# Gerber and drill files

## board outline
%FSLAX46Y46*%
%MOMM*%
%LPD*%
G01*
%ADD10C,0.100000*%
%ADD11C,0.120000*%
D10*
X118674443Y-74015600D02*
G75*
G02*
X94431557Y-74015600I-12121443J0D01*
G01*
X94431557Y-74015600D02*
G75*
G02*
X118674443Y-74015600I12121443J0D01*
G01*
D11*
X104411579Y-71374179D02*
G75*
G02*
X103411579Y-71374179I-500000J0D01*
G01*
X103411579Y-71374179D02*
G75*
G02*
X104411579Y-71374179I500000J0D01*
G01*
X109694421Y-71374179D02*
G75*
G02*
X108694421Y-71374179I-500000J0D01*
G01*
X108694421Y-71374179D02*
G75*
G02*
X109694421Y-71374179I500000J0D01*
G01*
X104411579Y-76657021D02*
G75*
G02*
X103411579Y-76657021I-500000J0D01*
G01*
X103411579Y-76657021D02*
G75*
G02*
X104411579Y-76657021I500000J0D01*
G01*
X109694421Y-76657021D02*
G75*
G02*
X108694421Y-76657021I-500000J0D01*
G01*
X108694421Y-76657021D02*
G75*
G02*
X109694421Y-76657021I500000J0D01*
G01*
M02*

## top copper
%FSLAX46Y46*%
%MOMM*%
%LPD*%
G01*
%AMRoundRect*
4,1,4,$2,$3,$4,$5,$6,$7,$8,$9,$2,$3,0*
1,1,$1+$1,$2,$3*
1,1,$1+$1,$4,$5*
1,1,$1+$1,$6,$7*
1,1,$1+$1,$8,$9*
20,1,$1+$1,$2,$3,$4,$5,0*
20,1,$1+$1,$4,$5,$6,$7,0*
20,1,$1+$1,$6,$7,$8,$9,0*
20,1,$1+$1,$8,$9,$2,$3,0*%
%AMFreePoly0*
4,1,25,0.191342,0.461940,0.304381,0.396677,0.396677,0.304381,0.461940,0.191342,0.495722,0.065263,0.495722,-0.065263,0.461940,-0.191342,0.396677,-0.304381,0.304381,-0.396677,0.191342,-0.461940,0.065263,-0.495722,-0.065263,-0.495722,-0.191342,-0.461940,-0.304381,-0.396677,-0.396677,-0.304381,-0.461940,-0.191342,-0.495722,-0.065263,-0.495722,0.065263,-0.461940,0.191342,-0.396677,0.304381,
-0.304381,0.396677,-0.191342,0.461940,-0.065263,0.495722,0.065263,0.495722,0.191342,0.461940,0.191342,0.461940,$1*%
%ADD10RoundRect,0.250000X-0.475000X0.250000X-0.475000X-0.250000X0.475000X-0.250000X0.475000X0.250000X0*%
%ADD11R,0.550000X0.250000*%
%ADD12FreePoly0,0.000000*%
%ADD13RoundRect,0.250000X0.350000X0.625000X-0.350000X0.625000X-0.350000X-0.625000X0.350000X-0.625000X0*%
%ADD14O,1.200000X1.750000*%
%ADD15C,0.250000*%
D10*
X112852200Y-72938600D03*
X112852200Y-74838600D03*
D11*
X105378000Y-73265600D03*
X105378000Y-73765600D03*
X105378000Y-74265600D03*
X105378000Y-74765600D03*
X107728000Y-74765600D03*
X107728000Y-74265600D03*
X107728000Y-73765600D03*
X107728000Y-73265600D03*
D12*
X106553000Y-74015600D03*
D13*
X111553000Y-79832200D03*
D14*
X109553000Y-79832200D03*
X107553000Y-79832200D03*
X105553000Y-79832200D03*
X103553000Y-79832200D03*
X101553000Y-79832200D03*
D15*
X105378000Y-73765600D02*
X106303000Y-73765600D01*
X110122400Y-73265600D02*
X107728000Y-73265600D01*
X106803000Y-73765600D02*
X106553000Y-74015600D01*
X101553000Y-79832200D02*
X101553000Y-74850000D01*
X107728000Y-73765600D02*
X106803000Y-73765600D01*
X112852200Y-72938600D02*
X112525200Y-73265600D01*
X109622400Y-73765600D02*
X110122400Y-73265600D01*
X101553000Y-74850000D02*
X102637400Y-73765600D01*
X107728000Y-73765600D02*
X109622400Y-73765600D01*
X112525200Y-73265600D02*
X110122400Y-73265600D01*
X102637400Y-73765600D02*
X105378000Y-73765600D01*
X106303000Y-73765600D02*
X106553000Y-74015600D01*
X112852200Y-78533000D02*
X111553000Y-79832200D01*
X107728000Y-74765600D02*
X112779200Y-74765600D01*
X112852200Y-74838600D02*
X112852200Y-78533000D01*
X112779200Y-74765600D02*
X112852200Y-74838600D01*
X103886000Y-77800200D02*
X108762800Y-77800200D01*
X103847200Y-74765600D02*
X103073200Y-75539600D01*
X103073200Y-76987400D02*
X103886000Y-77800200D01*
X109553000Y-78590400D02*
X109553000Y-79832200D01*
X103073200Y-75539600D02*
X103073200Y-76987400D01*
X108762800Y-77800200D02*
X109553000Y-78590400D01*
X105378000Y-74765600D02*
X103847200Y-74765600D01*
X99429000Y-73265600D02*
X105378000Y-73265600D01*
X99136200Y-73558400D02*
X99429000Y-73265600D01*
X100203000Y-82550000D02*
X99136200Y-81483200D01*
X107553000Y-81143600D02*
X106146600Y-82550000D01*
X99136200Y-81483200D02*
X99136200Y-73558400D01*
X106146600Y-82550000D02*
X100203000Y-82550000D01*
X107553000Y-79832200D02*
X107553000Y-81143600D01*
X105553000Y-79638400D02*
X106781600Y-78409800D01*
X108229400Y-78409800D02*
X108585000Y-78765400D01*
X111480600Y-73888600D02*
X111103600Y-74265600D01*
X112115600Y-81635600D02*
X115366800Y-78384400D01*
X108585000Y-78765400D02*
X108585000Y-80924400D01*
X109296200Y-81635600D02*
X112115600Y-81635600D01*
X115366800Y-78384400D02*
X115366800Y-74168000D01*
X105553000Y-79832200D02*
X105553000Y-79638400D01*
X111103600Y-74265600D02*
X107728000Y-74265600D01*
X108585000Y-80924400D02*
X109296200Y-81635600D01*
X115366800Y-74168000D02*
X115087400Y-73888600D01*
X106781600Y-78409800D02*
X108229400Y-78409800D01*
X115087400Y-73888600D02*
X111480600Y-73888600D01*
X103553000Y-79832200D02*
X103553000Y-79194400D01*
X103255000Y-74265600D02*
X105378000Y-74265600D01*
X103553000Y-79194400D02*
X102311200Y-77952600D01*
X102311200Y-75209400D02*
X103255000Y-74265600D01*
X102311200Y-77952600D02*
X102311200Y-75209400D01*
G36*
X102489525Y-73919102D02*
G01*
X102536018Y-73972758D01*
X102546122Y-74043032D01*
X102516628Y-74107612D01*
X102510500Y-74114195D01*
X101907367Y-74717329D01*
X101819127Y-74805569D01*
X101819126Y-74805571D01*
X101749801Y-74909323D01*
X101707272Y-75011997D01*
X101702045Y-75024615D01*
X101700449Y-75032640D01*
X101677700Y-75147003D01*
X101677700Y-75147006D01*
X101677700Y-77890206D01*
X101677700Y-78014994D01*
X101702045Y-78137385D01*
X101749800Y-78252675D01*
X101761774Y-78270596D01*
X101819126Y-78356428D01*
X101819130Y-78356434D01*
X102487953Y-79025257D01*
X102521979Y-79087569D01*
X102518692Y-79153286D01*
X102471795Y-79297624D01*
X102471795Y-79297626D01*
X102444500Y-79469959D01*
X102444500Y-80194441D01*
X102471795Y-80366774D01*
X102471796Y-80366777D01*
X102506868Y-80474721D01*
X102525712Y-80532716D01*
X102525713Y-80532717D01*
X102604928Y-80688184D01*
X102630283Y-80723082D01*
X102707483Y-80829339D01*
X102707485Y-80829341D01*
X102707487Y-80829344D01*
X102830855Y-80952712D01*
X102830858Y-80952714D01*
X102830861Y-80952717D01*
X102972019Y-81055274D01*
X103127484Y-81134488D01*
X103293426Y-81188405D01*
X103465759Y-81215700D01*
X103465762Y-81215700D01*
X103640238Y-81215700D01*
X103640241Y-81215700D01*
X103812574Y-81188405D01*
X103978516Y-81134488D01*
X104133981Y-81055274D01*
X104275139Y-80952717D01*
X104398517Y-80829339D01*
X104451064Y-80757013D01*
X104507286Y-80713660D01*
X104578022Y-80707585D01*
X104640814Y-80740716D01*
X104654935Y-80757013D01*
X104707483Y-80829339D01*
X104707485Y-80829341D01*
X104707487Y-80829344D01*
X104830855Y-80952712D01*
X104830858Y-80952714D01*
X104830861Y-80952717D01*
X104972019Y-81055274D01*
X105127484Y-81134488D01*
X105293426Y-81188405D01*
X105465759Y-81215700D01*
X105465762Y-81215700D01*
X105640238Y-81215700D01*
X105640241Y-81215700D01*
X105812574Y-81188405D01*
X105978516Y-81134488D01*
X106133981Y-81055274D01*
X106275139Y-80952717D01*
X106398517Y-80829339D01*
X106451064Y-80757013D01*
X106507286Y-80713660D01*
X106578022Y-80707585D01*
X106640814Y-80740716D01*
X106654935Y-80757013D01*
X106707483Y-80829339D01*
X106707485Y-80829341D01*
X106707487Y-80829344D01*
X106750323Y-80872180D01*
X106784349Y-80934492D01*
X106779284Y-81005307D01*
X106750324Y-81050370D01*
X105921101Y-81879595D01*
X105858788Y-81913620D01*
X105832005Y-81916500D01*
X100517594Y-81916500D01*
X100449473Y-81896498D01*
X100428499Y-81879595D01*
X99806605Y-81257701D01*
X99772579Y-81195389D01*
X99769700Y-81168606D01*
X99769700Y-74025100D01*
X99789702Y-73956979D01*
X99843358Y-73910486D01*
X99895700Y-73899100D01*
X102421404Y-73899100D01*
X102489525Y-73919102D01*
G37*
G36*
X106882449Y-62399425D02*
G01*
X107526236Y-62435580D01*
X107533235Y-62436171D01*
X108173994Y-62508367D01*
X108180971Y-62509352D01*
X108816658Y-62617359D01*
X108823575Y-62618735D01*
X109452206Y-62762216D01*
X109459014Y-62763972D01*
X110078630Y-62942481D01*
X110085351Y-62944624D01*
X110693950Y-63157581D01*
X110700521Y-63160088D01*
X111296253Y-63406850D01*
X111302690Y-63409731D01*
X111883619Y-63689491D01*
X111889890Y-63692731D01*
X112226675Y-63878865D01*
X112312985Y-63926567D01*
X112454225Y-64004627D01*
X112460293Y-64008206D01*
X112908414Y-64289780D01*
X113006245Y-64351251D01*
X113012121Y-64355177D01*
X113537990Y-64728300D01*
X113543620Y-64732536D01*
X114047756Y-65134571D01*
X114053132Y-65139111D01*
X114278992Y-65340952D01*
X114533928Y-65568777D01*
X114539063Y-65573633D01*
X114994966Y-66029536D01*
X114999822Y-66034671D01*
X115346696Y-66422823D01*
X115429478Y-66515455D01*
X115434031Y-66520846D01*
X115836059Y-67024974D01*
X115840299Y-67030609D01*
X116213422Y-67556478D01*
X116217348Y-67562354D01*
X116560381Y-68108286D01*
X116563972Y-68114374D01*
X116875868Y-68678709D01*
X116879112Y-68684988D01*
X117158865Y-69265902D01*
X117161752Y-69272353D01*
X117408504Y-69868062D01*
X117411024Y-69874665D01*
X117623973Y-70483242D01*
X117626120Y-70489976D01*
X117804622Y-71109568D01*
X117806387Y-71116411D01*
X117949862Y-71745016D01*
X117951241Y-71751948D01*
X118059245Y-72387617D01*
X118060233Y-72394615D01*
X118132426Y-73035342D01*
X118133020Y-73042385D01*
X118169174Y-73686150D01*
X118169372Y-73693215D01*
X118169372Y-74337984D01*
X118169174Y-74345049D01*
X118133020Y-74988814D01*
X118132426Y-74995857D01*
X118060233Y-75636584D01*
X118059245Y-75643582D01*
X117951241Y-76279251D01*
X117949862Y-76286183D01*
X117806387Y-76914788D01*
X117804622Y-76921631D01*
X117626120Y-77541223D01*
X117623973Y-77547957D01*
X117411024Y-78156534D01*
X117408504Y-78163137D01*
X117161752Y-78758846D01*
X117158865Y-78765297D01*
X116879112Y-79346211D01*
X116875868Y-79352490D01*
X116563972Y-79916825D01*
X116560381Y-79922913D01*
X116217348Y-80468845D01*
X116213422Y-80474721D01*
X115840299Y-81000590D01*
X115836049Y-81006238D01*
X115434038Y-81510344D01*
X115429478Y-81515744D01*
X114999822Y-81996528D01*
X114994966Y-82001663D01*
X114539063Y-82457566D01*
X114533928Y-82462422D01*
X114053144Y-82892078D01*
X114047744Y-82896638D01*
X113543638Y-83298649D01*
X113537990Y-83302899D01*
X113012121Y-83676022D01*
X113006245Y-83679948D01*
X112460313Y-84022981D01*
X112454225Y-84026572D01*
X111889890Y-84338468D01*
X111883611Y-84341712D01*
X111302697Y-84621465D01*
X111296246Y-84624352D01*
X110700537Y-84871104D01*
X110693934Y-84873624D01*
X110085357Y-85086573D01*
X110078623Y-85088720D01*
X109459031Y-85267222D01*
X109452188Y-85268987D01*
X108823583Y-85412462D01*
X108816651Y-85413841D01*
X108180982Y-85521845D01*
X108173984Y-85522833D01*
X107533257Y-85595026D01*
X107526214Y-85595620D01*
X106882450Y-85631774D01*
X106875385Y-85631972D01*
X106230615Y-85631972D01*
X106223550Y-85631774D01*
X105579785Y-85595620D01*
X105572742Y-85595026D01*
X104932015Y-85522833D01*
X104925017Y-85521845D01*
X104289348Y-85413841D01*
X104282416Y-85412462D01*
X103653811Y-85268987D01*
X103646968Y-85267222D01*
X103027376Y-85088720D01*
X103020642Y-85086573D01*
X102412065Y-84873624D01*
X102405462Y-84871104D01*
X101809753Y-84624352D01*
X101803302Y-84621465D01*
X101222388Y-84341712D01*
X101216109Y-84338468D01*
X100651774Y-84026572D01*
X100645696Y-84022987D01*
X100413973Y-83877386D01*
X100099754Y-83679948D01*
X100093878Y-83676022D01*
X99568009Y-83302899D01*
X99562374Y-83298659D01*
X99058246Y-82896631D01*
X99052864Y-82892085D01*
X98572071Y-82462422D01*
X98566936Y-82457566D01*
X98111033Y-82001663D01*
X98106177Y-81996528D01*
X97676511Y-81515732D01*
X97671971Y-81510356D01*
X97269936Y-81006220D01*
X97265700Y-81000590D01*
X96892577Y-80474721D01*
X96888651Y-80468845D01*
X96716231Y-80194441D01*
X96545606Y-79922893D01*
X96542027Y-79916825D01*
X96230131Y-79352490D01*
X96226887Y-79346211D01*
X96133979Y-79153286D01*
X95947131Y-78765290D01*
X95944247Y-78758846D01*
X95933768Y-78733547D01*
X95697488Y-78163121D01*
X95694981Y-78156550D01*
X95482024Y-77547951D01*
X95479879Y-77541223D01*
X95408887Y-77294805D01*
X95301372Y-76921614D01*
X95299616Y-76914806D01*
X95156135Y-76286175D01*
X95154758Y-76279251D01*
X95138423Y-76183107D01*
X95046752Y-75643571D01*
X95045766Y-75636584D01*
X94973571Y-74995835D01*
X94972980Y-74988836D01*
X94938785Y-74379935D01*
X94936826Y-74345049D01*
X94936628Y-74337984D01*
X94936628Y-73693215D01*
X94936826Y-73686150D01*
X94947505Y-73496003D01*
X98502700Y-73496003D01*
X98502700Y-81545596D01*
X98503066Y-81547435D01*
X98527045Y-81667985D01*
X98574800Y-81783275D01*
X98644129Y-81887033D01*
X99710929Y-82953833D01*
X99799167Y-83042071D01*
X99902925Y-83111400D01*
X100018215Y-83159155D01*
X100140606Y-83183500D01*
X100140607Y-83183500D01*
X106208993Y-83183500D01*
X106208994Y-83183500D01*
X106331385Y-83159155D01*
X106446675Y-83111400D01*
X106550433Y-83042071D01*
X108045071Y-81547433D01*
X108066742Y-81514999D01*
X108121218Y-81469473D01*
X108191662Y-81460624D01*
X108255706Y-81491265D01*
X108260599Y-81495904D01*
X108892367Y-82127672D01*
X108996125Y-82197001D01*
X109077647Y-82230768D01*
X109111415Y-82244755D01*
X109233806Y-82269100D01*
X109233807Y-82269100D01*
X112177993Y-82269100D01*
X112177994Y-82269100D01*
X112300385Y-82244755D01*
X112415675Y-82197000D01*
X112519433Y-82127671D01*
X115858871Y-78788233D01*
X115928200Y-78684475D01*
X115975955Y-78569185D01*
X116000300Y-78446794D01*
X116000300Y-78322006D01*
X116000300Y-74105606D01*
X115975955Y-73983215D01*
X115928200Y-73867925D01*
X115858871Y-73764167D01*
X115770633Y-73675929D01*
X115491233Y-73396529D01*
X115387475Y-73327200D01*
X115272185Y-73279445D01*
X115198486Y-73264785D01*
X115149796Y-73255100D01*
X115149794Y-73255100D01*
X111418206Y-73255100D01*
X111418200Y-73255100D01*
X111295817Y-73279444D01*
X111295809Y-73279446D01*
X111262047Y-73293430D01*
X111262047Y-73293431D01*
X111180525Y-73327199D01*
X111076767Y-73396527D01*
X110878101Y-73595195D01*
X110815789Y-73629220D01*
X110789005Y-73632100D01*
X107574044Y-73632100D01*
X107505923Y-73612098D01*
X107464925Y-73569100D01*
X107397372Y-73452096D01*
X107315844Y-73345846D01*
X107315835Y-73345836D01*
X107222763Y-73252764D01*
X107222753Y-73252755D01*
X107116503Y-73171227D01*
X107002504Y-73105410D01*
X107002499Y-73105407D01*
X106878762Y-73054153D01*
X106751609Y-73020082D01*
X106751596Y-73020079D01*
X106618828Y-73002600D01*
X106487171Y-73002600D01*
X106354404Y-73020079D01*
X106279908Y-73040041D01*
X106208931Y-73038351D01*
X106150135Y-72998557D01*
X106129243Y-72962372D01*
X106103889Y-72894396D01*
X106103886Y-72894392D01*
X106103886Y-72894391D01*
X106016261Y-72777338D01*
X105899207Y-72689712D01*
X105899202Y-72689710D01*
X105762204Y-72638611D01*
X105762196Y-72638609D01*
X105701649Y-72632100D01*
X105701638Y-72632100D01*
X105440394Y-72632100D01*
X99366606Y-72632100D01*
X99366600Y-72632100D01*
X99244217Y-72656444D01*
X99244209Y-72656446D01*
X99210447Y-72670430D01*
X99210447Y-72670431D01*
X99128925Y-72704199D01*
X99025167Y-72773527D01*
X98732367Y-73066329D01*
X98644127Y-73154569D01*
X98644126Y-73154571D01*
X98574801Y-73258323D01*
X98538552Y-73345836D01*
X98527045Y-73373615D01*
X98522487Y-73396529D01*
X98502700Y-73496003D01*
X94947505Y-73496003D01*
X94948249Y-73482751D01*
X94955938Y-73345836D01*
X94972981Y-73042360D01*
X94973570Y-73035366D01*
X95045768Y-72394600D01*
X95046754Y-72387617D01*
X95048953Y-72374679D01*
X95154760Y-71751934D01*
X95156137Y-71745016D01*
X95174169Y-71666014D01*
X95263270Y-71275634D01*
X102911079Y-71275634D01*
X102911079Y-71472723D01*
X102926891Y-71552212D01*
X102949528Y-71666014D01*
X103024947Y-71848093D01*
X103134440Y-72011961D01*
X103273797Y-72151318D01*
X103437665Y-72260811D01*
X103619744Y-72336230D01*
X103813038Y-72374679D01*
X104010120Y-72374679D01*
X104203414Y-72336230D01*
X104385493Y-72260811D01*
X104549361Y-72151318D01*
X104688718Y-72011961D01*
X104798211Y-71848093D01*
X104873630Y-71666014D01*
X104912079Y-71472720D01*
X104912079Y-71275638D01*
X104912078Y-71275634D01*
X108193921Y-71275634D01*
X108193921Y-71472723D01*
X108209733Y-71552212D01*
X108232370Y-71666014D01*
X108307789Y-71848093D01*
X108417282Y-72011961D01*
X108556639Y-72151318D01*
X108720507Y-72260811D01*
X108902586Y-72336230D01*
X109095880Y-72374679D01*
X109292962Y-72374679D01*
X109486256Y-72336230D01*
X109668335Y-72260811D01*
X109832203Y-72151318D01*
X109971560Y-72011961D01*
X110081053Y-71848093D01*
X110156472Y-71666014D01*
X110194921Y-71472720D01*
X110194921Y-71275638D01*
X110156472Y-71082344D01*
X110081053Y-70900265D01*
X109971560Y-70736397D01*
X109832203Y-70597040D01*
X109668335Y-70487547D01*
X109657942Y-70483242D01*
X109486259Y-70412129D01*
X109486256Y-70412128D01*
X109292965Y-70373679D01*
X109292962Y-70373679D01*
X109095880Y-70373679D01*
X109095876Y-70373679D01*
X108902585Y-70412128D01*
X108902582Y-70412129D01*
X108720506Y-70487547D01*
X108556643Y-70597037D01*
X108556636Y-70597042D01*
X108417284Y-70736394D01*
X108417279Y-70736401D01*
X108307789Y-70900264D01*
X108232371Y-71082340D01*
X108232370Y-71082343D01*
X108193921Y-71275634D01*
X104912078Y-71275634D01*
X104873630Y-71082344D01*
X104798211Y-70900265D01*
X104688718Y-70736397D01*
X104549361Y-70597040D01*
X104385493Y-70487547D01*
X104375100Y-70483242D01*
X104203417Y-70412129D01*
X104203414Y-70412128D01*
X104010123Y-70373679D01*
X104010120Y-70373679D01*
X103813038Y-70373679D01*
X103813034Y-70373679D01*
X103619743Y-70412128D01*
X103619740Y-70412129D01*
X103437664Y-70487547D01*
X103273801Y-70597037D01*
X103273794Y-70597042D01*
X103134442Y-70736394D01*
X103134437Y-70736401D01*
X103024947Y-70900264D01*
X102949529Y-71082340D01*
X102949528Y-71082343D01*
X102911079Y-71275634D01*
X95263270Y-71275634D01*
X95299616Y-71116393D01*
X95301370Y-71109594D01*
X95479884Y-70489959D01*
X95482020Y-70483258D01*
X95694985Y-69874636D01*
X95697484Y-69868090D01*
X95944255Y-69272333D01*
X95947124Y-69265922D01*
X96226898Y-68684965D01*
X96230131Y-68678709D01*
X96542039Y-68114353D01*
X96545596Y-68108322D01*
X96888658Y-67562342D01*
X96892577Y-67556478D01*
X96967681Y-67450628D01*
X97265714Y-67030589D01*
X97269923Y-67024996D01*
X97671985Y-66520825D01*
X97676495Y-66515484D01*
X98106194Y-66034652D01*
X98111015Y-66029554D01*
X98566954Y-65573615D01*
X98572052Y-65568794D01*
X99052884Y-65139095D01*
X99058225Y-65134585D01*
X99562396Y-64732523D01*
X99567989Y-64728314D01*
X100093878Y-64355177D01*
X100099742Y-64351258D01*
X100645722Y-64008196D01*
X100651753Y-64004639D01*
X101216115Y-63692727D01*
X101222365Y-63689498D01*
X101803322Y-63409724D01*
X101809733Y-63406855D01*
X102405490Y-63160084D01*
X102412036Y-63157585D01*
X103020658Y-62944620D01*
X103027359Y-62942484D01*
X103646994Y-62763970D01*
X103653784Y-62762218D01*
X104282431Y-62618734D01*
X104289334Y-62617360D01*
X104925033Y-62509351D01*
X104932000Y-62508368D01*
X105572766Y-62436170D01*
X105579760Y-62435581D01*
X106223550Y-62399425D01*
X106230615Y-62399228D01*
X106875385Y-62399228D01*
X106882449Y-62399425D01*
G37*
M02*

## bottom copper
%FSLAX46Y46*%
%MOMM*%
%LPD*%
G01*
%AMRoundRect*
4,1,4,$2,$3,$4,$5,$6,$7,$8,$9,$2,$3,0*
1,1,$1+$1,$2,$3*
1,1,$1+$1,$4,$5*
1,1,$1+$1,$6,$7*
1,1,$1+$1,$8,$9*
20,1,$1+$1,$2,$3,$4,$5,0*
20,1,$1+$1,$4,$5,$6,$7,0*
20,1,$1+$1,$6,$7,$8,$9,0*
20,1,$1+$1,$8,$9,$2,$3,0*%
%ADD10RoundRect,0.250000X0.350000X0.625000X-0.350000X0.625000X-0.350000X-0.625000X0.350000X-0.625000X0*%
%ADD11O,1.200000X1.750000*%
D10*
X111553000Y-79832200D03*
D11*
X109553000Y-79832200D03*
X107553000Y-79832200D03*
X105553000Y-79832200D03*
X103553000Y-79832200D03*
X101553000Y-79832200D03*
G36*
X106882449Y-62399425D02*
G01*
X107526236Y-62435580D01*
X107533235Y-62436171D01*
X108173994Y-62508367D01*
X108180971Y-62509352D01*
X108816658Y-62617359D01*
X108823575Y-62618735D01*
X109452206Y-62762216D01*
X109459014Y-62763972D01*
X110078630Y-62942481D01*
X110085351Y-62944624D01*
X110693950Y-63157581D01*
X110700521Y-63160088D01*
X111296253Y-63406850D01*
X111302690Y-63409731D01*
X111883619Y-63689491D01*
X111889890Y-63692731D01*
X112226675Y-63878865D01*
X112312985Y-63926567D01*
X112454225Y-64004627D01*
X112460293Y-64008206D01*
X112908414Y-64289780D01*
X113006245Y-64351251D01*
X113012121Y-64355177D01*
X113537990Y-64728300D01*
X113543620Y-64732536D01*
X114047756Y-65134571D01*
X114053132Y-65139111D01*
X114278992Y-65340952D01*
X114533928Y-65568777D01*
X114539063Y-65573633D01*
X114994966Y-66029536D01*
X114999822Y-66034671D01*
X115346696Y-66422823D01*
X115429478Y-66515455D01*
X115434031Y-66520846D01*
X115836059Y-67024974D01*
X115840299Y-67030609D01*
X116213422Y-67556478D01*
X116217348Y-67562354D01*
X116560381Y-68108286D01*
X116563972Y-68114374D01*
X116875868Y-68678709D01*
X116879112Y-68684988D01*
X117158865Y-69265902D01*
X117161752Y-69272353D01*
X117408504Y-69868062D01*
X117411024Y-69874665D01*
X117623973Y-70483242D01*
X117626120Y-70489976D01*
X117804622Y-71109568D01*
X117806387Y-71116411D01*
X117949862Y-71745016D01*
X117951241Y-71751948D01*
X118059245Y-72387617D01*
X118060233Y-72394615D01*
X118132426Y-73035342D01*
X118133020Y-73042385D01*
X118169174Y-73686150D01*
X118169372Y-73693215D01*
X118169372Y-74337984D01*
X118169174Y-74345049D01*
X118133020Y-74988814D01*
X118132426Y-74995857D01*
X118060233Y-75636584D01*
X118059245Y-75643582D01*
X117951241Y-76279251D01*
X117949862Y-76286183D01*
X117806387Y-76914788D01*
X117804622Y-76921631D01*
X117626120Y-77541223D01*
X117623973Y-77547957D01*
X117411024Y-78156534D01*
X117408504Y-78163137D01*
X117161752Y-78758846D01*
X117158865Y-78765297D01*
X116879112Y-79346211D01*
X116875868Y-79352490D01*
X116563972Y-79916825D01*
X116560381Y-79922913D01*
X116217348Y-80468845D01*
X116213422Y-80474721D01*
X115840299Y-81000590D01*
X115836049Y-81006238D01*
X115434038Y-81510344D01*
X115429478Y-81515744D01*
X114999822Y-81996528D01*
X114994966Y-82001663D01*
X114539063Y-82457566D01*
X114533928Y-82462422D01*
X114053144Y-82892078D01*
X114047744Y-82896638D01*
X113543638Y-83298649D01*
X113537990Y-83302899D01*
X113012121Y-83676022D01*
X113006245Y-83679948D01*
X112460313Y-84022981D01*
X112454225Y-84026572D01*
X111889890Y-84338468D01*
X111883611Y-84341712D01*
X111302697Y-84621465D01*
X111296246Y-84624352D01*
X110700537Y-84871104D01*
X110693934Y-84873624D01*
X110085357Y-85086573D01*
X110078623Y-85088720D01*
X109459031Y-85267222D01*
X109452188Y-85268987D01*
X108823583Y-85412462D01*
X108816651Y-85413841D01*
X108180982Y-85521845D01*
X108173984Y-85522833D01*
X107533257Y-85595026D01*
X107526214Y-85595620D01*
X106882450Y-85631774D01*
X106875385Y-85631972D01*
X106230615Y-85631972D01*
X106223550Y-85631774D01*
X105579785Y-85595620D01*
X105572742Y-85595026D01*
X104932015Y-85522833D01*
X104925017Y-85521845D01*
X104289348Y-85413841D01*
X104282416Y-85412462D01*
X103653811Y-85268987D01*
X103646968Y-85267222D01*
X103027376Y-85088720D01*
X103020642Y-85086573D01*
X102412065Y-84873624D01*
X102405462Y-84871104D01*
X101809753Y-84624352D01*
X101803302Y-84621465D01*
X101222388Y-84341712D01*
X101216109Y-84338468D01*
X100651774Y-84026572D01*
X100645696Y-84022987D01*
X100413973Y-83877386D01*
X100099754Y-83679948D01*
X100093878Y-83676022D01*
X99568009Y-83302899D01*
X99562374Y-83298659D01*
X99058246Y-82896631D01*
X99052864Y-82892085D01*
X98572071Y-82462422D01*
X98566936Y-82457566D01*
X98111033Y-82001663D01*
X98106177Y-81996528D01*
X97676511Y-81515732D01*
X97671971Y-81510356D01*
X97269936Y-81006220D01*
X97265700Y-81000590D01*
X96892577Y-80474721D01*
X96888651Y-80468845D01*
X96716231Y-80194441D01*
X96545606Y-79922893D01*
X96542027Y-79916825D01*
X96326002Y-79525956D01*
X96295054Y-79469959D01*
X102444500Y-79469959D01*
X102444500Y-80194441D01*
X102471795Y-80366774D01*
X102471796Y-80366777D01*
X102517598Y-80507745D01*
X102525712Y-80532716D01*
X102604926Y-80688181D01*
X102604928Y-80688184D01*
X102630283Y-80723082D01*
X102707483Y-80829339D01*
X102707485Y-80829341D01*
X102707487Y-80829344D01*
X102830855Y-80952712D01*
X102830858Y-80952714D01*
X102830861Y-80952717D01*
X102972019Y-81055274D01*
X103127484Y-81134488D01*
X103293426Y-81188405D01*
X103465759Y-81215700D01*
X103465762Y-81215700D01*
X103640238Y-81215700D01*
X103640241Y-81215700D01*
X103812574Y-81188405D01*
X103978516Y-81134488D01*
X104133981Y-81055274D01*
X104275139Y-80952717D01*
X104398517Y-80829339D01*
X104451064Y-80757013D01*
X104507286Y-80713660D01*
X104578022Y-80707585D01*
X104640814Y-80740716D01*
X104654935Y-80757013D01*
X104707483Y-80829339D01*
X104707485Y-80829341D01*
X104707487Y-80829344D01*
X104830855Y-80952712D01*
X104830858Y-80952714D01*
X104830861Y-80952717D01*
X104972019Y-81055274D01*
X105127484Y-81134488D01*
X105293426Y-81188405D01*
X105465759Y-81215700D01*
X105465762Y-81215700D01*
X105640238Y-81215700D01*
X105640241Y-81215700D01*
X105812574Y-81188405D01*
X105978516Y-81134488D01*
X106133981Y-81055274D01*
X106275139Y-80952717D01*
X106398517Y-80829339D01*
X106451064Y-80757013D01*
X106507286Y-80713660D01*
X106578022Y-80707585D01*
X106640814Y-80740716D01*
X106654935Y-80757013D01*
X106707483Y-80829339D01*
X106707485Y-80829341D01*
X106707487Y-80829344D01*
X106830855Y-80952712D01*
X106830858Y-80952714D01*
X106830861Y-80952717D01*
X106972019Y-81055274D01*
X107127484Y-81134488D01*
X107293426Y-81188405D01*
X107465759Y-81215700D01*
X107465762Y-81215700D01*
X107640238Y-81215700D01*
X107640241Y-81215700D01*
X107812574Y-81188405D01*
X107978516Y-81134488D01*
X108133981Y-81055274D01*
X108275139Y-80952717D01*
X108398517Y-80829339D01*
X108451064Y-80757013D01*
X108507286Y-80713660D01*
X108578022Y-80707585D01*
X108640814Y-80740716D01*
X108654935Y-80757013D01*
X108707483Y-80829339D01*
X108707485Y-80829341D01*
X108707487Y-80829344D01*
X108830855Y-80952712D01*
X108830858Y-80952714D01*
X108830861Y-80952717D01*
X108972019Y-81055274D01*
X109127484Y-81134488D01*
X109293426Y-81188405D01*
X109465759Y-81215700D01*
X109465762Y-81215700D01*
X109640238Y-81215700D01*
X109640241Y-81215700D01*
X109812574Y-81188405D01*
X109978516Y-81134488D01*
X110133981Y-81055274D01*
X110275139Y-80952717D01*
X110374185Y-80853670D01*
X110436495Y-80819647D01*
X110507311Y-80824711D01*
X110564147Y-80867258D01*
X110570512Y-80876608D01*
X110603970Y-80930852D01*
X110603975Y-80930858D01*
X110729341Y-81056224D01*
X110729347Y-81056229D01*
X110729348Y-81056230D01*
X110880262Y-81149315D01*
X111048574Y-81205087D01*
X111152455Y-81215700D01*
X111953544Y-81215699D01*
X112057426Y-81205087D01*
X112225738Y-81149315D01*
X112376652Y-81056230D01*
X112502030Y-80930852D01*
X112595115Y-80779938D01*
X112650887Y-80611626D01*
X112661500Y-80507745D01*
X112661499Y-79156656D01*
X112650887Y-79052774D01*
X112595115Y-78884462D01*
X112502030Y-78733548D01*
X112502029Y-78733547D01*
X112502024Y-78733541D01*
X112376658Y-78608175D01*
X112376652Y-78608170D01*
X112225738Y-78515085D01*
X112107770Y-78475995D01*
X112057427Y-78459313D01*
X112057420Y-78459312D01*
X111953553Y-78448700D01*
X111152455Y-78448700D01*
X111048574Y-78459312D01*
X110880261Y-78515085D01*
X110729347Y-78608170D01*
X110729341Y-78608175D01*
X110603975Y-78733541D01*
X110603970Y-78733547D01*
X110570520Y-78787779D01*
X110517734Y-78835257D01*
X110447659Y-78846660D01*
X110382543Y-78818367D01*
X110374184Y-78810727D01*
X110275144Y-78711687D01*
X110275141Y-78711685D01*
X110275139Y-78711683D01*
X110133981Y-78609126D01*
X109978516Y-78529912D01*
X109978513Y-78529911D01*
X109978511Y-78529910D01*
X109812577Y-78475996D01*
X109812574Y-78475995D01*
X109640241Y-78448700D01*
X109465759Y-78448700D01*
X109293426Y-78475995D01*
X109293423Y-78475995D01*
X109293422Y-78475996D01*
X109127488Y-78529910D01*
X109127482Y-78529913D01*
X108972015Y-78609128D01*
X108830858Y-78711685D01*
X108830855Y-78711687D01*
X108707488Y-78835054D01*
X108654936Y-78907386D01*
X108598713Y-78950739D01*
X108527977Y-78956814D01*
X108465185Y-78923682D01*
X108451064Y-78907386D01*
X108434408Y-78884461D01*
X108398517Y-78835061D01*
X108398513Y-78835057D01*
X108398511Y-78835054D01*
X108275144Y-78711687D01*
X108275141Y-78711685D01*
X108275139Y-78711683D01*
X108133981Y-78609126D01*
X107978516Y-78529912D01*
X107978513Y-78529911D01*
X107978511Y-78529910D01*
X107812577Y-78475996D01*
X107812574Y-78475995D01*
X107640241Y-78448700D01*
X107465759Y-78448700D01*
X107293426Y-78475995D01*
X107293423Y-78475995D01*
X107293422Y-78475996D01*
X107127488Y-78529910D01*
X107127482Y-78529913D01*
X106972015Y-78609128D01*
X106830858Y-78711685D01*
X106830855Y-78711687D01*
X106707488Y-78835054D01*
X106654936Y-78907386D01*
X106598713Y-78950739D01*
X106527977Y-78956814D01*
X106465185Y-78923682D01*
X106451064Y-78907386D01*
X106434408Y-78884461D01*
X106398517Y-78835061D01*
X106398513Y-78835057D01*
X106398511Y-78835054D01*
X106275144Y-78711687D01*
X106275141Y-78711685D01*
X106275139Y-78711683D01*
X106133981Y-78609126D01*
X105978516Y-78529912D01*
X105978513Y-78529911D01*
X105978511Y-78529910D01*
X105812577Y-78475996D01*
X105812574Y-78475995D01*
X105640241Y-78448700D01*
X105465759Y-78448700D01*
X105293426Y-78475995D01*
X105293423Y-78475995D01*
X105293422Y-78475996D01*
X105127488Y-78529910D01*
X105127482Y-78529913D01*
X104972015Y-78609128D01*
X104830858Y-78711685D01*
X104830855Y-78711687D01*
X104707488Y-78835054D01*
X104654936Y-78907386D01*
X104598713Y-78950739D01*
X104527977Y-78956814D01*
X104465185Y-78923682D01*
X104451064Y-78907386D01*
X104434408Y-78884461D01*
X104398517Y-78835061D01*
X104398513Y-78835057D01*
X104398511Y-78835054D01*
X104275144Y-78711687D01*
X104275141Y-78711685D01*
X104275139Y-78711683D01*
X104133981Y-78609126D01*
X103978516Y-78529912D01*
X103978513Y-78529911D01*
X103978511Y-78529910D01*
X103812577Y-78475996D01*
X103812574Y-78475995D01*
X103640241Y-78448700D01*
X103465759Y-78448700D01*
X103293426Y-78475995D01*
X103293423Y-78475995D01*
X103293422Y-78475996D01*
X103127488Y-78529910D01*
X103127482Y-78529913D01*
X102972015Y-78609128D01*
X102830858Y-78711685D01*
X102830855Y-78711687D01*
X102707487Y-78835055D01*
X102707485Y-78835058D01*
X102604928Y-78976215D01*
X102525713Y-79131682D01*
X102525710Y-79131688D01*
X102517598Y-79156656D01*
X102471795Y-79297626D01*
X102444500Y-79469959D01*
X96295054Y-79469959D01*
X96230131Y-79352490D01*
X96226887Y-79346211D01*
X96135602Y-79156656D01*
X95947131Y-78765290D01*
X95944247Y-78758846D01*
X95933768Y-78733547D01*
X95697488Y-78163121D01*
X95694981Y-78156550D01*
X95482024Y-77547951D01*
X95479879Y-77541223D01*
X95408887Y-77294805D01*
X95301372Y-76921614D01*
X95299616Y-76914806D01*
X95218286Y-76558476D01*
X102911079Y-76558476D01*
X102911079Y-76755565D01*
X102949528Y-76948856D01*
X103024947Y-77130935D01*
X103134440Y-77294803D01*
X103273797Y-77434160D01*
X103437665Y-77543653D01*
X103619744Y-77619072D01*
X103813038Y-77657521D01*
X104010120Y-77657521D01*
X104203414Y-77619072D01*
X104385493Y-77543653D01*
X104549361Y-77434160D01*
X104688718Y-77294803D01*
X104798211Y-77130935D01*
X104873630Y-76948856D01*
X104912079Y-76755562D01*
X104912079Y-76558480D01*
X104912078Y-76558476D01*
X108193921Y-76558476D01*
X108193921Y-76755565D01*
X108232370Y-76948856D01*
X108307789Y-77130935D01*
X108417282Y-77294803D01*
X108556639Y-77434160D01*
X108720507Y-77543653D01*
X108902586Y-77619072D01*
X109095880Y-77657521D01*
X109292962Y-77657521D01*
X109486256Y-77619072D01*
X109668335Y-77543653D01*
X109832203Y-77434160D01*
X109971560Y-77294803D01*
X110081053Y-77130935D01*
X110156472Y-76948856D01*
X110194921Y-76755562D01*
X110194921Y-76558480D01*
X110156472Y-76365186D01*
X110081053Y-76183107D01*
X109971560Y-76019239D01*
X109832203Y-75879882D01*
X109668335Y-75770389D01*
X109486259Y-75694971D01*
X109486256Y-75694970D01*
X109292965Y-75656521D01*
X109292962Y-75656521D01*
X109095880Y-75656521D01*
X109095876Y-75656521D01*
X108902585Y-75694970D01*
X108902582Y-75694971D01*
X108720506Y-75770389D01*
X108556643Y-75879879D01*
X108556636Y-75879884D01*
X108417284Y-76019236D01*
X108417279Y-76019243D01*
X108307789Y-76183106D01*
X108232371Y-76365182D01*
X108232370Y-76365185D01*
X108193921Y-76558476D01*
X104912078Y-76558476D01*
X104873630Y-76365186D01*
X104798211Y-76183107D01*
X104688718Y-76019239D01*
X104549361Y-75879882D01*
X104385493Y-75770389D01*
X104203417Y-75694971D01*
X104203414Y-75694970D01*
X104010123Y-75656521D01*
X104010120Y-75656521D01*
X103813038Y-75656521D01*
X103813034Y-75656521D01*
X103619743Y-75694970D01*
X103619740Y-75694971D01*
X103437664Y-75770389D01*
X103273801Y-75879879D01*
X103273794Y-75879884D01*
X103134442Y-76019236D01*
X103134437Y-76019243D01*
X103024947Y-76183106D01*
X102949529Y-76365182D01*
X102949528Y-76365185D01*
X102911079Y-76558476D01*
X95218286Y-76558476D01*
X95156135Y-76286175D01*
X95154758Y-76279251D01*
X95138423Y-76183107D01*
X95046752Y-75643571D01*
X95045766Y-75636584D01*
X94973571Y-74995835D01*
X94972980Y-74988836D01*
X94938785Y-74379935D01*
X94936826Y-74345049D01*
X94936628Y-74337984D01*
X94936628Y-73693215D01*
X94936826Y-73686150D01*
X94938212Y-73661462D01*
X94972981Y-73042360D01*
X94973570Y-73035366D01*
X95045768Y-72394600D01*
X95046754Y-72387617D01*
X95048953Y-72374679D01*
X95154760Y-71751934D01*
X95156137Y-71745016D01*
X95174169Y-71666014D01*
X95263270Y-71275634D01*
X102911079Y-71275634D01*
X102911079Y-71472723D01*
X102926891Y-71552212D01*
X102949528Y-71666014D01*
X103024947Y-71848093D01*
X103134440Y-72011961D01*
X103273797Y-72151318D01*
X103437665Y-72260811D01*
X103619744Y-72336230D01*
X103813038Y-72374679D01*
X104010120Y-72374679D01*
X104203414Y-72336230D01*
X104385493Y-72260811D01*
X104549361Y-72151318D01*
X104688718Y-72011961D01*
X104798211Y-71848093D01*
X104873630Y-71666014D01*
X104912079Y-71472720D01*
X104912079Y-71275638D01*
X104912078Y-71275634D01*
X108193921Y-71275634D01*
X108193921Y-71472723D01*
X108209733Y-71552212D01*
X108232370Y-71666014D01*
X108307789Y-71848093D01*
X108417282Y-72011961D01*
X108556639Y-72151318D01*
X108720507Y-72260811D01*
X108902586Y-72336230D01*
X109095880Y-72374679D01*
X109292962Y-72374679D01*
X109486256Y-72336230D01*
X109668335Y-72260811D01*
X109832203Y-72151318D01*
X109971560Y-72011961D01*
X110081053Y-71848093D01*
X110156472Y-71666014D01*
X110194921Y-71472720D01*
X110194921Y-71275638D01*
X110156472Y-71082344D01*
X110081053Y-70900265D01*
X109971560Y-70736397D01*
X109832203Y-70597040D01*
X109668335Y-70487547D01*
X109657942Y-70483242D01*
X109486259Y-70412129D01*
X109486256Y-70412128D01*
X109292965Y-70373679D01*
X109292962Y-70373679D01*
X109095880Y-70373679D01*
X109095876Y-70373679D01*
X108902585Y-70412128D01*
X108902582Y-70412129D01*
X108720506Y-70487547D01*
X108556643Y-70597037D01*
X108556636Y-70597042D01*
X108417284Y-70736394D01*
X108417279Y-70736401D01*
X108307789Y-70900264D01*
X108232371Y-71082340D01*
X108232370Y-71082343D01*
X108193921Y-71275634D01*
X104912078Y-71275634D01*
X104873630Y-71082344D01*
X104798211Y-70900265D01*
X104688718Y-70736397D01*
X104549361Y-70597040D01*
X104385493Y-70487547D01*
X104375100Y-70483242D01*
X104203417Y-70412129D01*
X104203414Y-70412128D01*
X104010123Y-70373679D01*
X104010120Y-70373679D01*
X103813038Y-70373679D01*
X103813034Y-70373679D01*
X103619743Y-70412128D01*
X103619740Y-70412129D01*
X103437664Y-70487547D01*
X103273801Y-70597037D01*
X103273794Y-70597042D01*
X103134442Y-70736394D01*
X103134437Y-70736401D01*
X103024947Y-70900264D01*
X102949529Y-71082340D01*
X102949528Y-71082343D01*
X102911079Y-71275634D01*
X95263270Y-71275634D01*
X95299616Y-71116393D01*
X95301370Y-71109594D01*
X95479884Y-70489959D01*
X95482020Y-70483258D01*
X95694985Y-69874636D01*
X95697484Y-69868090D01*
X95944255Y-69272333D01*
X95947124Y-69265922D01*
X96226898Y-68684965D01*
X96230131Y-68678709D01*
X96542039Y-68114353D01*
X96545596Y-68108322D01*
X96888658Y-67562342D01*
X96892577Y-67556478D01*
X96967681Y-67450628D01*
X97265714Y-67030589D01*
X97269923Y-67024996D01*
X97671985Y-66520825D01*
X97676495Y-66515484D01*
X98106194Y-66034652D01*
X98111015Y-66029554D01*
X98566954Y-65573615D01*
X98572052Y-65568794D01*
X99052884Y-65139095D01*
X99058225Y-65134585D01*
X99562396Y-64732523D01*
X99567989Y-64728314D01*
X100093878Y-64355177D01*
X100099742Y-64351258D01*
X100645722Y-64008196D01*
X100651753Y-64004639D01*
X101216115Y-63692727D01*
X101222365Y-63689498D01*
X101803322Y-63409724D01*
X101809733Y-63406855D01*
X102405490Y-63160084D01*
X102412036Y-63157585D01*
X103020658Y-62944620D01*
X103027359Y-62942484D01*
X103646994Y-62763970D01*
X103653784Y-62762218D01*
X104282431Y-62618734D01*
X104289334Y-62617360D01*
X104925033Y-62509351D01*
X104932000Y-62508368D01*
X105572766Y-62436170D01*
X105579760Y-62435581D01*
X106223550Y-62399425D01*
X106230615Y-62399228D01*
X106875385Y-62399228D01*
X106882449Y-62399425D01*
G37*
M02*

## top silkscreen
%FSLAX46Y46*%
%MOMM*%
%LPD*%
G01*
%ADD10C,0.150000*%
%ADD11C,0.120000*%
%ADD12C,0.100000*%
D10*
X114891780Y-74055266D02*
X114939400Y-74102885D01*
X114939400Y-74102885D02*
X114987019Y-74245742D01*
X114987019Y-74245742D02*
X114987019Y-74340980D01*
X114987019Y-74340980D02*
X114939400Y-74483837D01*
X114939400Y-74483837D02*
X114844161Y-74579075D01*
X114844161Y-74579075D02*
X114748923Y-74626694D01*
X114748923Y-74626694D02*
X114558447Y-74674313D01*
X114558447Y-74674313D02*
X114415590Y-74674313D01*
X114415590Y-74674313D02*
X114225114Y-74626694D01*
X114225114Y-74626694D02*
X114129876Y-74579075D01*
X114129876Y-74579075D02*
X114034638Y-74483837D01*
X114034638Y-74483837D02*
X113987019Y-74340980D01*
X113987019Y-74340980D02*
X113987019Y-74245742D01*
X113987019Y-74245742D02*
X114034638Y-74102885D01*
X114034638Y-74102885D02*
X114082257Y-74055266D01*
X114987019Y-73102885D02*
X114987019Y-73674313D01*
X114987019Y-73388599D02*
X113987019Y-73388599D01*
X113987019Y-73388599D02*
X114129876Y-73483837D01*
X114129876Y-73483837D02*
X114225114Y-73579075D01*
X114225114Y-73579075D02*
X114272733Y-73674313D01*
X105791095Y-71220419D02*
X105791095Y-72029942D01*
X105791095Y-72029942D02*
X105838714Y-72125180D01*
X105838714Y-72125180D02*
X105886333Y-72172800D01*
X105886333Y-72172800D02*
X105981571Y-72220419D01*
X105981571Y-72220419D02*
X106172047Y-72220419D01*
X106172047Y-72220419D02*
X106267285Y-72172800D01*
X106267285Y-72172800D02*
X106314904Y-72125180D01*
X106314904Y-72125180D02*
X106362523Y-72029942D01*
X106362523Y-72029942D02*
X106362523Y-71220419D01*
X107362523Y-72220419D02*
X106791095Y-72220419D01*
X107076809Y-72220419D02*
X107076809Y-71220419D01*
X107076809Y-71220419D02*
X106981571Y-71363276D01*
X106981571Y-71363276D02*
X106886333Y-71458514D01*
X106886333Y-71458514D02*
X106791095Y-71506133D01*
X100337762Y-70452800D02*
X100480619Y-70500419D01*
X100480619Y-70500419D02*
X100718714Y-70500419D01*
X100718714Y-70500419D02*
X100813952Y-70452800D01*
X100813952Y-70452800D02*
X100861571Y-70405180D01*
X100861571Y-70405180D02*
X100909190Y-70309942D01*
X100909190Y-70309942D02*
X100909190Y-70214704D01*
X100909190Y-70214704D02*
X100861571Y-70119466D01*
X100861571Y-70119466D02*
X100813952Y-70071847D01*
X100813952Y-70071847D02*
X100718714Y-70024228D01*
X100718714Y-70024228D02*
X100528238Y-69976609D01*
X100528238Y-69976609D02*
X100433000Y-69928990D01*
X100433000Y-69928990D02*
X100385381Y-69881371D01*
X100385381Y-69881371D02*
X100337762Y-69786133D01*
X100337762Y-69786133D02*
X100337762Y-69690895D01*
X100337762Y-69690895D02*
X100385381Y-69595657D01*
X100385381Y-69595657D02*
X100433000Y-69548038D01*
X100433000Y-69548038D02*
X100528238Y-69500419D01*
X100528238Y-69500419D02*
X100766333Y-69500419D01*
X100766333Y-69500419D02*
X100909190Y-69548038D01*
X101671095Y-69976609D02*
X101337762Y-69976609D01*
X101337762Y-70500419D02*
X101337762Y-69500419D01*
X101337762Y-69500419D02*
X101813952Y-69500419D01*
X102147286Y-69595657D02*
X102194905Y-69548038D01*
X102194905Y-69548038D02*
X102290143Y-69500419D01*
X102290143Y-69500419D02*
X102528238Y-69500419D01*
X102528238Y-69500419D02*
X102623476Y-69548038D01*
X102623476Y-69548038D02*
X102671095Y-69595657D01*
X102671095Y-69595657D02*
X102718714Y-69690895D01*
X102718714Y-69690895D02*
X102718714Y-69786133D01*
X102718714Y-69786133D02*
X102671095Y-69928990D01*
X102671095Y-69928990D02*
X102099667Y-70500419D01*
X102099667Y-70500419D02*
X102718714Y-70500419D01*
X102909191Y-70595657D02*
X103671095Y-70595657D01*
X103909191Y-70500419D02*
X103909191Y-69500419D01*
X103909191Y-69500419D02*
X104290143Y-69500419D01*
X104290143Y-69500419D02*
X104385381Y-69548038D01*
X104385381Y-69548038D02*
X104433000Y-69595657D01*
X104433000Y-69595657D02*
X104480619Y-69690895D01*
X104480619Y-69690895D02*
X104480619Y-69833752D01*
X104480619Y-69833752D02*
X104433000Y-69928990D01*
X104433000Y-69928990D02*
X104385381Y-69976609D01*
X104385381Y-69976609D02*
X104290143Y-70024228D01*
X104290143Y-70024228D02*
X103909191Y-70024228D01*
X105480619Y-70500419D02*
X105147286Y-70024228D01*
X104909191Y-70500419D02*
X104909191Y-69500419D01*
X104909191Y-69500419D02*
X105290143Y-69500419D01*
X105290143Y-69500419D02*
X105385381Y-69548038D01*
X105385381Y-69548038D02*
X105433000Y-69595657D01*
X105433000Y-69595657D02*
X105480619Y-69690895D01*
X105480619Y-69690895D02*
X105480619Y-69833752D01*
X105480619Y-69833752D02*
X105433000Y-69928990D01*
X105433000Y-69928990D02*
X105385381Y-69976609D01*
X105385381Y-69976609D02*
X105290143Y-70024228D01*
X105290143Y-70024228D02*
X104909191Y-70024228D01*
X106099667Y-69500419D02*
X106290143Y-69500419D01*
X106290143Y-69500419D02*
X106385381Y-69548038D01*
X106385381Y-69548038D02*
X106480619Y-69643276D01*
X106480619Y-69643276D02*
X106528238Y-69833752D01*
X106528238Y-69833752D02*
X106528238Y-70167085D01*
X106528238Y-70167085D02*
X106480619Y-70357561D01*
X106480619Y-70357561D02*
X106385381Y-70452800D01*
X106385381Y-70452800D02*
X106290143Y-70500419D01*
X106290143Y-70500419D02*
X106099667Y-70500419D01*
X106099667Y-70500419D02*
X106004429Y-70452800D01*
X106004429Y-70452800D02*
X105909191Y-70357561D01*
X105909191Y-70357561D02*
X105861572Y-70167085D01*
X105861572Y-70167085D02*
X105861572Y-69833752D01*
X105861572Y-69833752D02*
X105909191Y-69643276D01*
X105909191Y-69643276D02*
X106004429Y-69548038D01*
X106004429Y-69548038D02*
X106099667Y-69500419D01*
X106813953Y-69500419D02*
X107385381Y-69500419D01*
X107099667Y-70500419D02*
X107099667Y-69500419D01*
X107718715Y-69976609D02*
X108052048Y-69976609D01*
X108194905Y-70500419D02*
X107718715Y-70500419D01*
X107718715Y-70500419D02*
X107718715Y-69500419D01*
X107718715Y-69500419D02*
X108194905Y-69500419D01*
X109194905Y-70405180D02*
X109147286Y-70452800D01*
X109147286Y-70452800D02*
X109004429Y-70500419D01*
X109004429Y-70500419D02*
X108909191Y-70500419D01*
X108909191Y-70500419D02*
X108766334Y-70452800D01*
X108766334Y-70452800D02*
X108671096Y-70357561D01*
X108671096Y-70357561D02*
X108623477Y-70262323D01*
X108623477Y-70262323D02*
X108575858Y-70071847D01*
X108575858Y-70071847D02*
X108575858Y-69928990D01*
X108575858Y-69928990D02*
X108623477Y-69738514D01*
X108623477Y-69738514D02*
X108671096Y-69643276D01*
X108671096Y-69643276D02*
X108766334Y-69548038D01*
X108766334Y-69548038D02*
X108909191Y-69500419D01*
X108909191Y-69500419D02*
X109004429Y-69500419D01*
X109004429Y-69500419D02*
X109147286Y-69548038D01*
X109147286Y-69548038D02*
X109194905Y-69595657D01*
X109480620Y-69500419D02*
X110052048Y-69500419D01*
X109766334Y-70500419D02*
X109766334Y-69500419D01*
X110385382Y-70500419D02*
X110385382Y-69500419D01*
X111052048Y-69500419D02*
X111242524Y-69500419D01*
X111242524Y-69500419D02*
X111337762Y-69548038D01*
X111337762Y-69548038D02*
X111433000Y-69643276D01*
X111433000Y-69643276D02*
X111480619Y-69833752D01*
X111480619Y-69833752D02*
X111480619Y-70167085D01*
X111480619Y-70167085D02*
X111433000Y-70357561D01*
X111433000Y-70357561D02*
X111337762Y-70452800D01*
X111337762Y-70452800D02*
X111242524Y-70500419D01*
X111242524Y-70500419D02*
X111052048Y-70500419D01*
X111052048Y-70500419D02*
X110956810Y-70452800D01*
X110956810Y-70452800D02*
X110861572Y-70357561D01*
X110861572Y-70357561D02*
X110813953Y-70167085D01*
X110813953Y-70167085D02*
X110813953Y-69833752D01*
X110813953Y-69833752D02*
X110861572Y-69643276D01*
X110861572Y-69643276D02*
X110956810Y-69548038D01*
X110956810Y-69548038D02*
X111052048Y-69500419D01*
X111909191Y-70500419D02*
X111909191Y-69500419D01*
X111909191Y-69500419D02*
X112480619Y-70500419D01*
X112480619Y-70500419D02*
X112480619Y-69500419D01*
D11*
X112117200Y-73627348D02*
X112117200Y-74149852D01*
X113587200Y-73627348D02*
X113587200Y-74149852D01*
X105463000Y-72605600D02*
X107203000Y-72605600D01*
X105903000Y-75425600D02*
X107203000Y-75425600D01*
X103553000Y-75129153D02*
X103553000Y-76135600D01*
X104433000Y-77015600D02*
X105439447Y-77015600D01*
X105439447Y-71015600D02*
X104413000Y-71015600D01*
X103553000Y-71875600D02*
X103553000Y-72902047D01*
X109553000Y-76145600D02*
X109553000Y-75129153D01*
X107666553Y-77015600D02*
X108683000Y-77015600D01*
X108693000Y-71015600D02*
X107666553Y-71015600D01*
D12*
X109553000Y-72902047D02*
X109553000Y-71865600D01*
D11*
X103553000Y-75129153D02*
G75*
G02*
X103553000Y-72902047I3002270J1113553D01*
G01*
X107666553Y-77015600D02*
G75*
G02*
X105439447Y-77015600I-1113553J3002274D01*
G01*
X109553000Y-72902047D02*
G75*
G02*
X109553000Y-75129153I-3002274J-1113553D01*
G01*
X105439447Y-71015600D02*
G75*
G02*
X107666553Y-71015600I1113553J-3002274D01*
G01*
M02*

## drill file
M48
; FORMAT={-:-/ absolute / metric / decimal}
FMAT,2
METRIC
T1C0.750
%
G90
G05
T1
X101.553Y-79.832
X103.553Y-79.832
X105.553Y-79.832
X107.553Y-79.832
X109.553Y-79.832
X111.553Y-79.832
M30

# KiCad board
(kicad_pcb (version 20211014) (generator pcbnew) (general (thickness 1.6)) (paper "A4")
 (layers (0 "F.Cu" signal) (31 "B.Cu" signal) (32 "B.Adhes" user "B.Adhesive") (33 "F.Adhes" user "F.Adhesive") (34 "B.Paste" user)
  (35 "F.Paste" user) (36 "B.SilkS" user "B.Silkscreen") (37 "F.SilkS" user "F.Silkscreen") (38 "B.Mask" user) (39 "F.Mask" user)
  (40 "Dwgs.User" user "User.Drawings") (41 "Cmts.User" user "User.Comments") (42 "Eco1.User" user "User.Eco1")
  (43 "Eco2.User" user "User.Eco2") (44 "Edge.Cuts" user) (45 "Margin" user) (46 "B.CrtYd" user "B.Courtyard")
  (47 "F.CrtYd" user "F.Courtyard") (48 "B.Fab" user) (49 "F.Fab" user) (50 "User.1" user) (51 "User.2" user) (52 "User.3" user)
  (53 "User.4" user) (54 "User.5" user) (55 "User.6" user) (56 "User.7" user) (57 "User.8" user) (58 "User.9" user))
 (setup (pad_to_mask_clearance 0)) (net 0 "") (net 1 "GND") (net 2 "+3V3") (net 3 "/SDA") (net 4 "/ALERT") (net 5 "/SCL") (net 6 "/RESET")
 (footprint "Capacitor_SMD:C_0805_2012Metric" (layer "F.Cu") (at 112.8522 73.8886 -90)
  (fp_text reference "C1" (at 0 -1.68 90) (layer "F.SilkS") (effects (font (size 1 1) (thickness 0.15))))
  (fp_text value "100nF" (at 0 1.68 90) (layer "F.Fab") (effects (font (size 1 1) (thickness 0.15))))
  (fp_line (start -0.261252 0.735) (end 0.261252 0.735) (layer "F.SilkS") (width 0.12))
  (fp_line (start -0.261252 -0.735) (end 0.261252 -0.735) (layer "F.SilkS") (width 0.12))
  (pad "1" smd roundrect (at -0.95 0 270) (size 1 1.45) (layers "F.Cu" "F.Paste" "F.Mask") (roundrect_rratio 0.25) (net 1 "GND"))
  (pad "2" smd roundrect (at 0.95 0 270) (size 1 1.45) (layers "F.Cu" "F.Paste" "F.Mask") (roundrect_rratio 0.25) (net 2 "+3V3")))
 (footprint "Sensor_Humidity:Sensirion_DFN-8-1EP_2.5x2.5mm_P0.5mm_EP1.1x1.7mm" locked (layer "F.Cu") (at 106.553 74.0156)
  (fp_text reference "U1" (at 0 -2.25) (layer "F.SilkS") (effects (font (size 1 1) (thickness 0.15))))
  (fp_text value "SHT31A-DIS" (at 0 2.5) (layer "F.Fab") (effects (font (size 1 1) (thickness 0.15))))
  (fp_line (start -1.09 -1.41) (end 0.65 -1.41) (layer "F.SilkS") (width 0.12))
  (fp_line (start -0.65 1.41) (end 0.65 1.41) (layer "F.SilkS") (width 0.12))
  (pad "" smd custom locked (at 0 0) (size 0.9 0.9) (layers "F.Paste") (zone_connect 0) (options (clearance outline) (anchor rect))
   (primitives))
  (pad "1" smd rect locked (at -1.175 -0.75) (size 0.55 0.25) (layers "F.Cu" "F.Paste" "F.Mask") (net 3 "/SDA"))
  (pad "2" smd rect locked (at -1.175 -0.25) (size 0.55 0.25) (layers "F.Cu" "F.Paste" "F.Mask") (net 1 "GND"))
  (pad "3" smd rect locked (at -1.175 0.25) (size 0.55 0.25) (layers "F.Cu" "F.Paste" "F.Mask") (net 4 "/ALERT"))
  (pad "4" smd rect locked (at -1.175 0.75 180) (size 0.55 0.25) (layers "F.Cu" "F.Paste" "F.Mask") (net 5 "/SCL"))
  (pad "5" smd rect locked (at 1.175 0.75) (size 0.55 0.25) (layers "F.Cu" "F.Paste" "F.Mask") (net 2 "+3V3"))
  (pad "6" smd rect locked (at 1.175 0.25) (size 0.55 0.25) (layers "F.Cu" "F.Paste" "F.Mask") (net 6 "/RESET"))
  (pad "7" smd rect locked (at 1.175 -0.25) (size 0.55 0.25) (layers "F.Cu" "F.Paste" "F.Mask") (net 1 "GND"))
  (pad "8" smd rect locked (at 1.175 -0.75) (size 0.55 0.25) (layers "F.Cu" "F.Paste" "F.Mask") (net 1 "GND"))
  (pad "9" smd custom locked (at 0 0) (size 1 1) (layers "F.Cu" "F.Mask") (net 1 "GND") (zone_connect 0)
   (options (clearance outline) (anchor circle)) (primitives)))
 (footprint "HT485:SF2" (layer "F.Cu") (at 106.553 74.0156)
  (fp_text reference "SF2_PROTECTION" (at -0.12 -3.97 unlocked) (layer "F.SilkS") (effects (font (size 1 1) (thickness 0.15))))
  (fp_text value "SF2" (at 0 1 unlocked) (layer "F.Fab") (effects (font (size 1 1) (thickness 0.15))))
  (fp_line (start -3 1.113553) (end -3 2.12) (layer "F.SilkS") (width 0.12))
  (fp_line (start -2.12 3) (end -1.113553 3) (layer "F.SilkS") (width 0.12))
  (fp_line (start -1.113553 -3) (end -2.14 -3) (layer "F.SilkS") (width 0.12))
  (fp_line (start -3 -2.14) (end -3 -1.113553) (layer "F.SilkS") (width 0.12))
  (fp_line (start 3 2.13) (end 3 1.113553) (layer "F.SilkS") (width 0.12))
  (fp_line (start 1.113553 3) (end 2.13 3) (layer "F.SilkS") (width 0.12))
  (fp_line (start 2.14 -3) (end 1.113553 -3) (layer "F.SilkS") (width 0.12))
  (fp_line (start 3 -1.113553) (end 3 -2.15) (layer "F.SilkS") (width 0.1))
  (fp_arc (start -3 1.113553) (mid -3.199858 0) (end -3 -1.113553) (layer "F.SilkS") (width 0.12))
  (fp_arc (start 1.113553 3) (mid 0 3.199858) (end -1.113553 3) (layer "F.SilkS") (width 0.12))
  (fp_arc (start 3 -1.113553) (mid 3.199858 0) (end 3 1.113553) (layer "F.SilkS") (width 0.12))
  (fp_arc (start -1.113553 -3) (mid 0 -3.199858) (end 1.113553 -3) (layer "F.SilkS") (width 0.12))
  (fp_circle (center -2.641421 -2.641421) (end -2.141421 -2.641421) (layer "Edge.Cuts") (width 0.12) (fill none))
  (fp_circle (center 2.641421 -2.641421) (end 3.141421 -2.641421) (layer "Edge.Cuts") (width 0.12) (fill none))
  (fp_circle (center -2.641421 2.641421) (end -2.141421 2.641421) (layer "Edge.Cuts") (width 0.12) (fill none))
  (fp_circle (center 2.641421 2.641421) (end 3.141421 2.641421) (layer "Edge.Cuts") (width 0.12) (fill none)))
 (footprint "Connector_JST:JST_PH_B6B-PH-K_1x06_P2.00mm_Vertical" (layer "B.Cu") (at 111.553 79.8322 180)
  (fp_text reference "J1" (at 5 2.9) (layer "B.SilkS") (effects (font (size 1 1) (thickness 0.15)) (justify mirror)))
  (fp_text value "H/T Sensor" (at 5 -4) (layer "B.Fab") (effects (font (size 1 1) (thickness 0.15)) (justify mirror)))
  (pad "1" thru_hole roundrect (at 0 0 180) (size 1.2 1.75) (drill 0.75) (layers *.Cu *.Mask) (roundrect_rratio 0.2083333333) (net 2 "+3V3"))
  (pad "2" thru_hole oval (at 2 0 180) (size 1.2 1.75) (drill 0.75) (layers *.Cu *.Mask) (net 5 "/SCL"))
  (pad "3" thru_hole oval (at 4 0 180) (size 1.2 1.75) (drill 0.75) (layers *.Cu *.Mask) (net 3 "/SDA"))
  (pad "4" thru_hole oval (at 6 0 180) (size 1.2 1.75) (drill 0.75) (layers *.Cu *.Mask) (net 6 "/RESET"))
  (pad "5" thru_hole oval (at 8 0 180) (size 1.2 1.75) (drill 0.75) (layers *.Cu *.Mask) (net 4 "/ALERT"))
  (pad "6" thru_hole oval (at 10 0 180) (size 1.2 1.75) (drill 0.75) (layers *.Cu *.Mask) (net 1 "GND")))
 (gr_circle locked (center 106.553 74.0156) (end 113.919 83.6422) (layer "Edge.Cuts") (width 0.1) (fill none))
 (segment (start 105.378 73.7656) (end 106.303 73.7656) (width 0.25) (layer "F.Cu") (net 1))
 (segment (start 110.1224 73.2656) (end 107.728 73.2656) (width 0.25) (layer "F.Cu") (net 1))
 (segment (start 106.803 73.7656) (end 106.553 74.0156) (width 0.25) (layer "F.Cu") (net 1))
 (segment (start 101.553 79.8322) (end 101.553 74.85) (width 0.25) (layer "F.Cu") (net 1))
 (segment (start 107.728 73.7656) (end 106.803 73.7656) (width 0.25) (layer "F.Cu") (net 1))
 (segment (start 112.8522 72.9386) (end 112.5252 73.2656) (width 0.25) (layer "F.Cu") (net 1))
 (segment (start 109.6224 73.7656) (end 110.1224 73.2656) (width 0.25) (layer "F.Cu") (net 1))
 (segment (start 101.553 74.85) (end 102.6374 73.7656) (width 0.25) (layer "F.Cu") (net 1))
 (segment (start 107.728 73.7656) (end 109.6224 73.7656) (width 0.25) (layer "F.Cu") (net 1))
 (segment (start 112.5252 73.2656) (end 110.1224 73.2656) (width 0.25) (layer "F.Cu") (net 1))
 (segment (start 102.6374 73.7656) (end 105.378 73.7656) (width 0.25) (layer "F.Cu") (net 1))
 (segment (start 106.303 73.7656) (end 106.553 74.0156) (width 0.25) (layer "F.Cu") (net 1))
 (segment (start 112.8522 78.533) (end 111.553 79.8322) (width 0.25) (layer "F.Cu") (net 2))
 (segment (start 107.728 74.7656) (end 112.7792 74.7656) (width 0.25) (layer "F.Cu") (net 2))
 (segment (start 112.8522 74.8386) (end 112.8522 78.533) (width 0.25) (layer "F.Cu") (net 2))
 (segment (start 112.7792 74.7656) (end 112.8522 74.8386) (width 0.25) (layer "F.Cu") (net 2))
 (segment (start 103.886 77.8002) (end 108.7628 77.8002) (width 0.25) (layer "F.Cu") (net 5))
 (segment (start 103.8472 74.7656) (end 103.0732 75.5396) (width 0.25) (layer "F.Cu") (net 5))
 (segment (start 103.0732 76.9874) (end 103.886 77.8002) (width 0.25) (layer "F.Cu") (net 5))
 (segment (start 109.553 78.5904) (end 109.553 79.8322) (width 0.25) (layer "F.Cu") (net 5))
 (segment (start 103.0732 75.5396) (end 103.0732 76.9874) (width 0.25) (layer "F.Cu") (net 5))
 (segment (start 108.7628 77.8002) (end 109.553 78.5904) (width 0.25) (layer "F.Cu") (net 5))
 (segment (start 105.378 74.7656) (end 103.8472 74.7656) (width 0.25) (layer "F.Cu") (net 5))
 (segment (start 99.429 73.2656) (end 105.378 73.2656) (width 0.25) (layer "F.Cu") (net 3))
 (segment (start 99.1362 73.5584) (end 99.429 73.2656) (width 0.25) (layer "F.Cu") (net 3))
 (segment (start 100.203 82.55) (end 99.1362 81.4832) (width 0.25) (layer "F.Cu") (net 3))
 (segment (start 107.553 81.1436) (end 106.1466 82.55) (width 0.25) (layer "F.Cu") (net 3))
 (segment (start 99.1362 81.4832) (end 99.1362 73.5584) (width 0.25) (layer "F.Cu") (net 3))
 (segment (start 106.1466 82.55) (end 100.203 82.55) (width 0.25) (layer "F.Cu") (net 3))
 (segment (start 107.553 79.8322) (end 107.553 81.1436) (width 0.25) (layer "F.Cu") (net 3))
 (segment (start 105.553 79.6384) (end 106.7816 78.4098) (width 0.25) (layer "F.Cu") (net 6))
 (segment (start 108.2294 78.4098) (end 108.585 78.7654) (width 0.25) (layer "F.Cu") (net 6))
 (segment (start 111.4806 73.8886) (end 111.1036 74.2656) (width 0.25) (layer "F.Cu") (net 6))
 (segment (start 112.1156 81.6356) (end 115.3668 78.3844) (width 0.25) (layer "F.Cu") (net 6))
 (segment (start 108.585 78.7654) (end 108.585 80.9244) (width 0.25) (layer "F.Cu") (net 6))
 (segment (start 109.2962 81.6356) (end 112.1156 81.6356) (width 0.25) (layer "F.Cu") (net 6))
 (segment (start 115.3668 78.3844) (end 115.3668 74.168) (width 0.25) (layer "F.Cu") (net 6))
 (segment (start 105.553 79.8322) (end 105.553 79.6384) (width 0.25) (layer "F.Cu") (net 6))
 (segment (start 111.1036 74.2656) (end 107.728 74.2656) (width 0.25) (layer "F.Cu") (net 6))
 (segment (start 108.585 80.9244) (end 109.2962 81.6356) (width 0.25) (layer "F.Cu") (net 6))
 (segment (start 115.3668 74.168) (end 115.0874 73.8886) (width 0.25) (layer "F.Cu") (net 6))
 (segment (start 106.7816 78.4098) (end 108.2294 78.4098) (width 0.25) (layer "F.Cu") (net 6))
 (segment (start 115.0874 73.8886) (end 111.4806 73.8886) (width 0.25) (layer "F.Cu") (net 6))
 (segment (start 103.553 79.8322) (end 103.553 79.1944) (width 0.25) (layer "F.Cu") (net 4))
 (segment (start 103.255 74.2656) (end 105.378 74.2656) (width 0.25) (layer "F.Cu") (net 4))
 (segment (start 103.553 79.1944) (end 102.3112 77.9526) (width 0.25) (layer "F.Cu") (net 4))
 (segment (start 102.3112 75.2094) (end 103.255 74.2656) (width 0.25) (layer "F.Cu") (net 4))
 (segment (start 102.3112 77.9526) (end 102.3112 75.2094) (width 0.25) (layer "F.Cu") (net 4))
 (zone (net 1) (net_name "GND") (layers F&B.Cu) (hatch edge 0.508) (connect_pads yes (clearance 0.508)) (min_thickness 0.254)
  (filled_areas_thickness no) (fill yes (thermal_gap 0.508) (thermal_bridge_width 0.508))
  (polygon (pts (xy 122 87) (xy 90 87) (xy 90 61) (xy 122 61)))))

